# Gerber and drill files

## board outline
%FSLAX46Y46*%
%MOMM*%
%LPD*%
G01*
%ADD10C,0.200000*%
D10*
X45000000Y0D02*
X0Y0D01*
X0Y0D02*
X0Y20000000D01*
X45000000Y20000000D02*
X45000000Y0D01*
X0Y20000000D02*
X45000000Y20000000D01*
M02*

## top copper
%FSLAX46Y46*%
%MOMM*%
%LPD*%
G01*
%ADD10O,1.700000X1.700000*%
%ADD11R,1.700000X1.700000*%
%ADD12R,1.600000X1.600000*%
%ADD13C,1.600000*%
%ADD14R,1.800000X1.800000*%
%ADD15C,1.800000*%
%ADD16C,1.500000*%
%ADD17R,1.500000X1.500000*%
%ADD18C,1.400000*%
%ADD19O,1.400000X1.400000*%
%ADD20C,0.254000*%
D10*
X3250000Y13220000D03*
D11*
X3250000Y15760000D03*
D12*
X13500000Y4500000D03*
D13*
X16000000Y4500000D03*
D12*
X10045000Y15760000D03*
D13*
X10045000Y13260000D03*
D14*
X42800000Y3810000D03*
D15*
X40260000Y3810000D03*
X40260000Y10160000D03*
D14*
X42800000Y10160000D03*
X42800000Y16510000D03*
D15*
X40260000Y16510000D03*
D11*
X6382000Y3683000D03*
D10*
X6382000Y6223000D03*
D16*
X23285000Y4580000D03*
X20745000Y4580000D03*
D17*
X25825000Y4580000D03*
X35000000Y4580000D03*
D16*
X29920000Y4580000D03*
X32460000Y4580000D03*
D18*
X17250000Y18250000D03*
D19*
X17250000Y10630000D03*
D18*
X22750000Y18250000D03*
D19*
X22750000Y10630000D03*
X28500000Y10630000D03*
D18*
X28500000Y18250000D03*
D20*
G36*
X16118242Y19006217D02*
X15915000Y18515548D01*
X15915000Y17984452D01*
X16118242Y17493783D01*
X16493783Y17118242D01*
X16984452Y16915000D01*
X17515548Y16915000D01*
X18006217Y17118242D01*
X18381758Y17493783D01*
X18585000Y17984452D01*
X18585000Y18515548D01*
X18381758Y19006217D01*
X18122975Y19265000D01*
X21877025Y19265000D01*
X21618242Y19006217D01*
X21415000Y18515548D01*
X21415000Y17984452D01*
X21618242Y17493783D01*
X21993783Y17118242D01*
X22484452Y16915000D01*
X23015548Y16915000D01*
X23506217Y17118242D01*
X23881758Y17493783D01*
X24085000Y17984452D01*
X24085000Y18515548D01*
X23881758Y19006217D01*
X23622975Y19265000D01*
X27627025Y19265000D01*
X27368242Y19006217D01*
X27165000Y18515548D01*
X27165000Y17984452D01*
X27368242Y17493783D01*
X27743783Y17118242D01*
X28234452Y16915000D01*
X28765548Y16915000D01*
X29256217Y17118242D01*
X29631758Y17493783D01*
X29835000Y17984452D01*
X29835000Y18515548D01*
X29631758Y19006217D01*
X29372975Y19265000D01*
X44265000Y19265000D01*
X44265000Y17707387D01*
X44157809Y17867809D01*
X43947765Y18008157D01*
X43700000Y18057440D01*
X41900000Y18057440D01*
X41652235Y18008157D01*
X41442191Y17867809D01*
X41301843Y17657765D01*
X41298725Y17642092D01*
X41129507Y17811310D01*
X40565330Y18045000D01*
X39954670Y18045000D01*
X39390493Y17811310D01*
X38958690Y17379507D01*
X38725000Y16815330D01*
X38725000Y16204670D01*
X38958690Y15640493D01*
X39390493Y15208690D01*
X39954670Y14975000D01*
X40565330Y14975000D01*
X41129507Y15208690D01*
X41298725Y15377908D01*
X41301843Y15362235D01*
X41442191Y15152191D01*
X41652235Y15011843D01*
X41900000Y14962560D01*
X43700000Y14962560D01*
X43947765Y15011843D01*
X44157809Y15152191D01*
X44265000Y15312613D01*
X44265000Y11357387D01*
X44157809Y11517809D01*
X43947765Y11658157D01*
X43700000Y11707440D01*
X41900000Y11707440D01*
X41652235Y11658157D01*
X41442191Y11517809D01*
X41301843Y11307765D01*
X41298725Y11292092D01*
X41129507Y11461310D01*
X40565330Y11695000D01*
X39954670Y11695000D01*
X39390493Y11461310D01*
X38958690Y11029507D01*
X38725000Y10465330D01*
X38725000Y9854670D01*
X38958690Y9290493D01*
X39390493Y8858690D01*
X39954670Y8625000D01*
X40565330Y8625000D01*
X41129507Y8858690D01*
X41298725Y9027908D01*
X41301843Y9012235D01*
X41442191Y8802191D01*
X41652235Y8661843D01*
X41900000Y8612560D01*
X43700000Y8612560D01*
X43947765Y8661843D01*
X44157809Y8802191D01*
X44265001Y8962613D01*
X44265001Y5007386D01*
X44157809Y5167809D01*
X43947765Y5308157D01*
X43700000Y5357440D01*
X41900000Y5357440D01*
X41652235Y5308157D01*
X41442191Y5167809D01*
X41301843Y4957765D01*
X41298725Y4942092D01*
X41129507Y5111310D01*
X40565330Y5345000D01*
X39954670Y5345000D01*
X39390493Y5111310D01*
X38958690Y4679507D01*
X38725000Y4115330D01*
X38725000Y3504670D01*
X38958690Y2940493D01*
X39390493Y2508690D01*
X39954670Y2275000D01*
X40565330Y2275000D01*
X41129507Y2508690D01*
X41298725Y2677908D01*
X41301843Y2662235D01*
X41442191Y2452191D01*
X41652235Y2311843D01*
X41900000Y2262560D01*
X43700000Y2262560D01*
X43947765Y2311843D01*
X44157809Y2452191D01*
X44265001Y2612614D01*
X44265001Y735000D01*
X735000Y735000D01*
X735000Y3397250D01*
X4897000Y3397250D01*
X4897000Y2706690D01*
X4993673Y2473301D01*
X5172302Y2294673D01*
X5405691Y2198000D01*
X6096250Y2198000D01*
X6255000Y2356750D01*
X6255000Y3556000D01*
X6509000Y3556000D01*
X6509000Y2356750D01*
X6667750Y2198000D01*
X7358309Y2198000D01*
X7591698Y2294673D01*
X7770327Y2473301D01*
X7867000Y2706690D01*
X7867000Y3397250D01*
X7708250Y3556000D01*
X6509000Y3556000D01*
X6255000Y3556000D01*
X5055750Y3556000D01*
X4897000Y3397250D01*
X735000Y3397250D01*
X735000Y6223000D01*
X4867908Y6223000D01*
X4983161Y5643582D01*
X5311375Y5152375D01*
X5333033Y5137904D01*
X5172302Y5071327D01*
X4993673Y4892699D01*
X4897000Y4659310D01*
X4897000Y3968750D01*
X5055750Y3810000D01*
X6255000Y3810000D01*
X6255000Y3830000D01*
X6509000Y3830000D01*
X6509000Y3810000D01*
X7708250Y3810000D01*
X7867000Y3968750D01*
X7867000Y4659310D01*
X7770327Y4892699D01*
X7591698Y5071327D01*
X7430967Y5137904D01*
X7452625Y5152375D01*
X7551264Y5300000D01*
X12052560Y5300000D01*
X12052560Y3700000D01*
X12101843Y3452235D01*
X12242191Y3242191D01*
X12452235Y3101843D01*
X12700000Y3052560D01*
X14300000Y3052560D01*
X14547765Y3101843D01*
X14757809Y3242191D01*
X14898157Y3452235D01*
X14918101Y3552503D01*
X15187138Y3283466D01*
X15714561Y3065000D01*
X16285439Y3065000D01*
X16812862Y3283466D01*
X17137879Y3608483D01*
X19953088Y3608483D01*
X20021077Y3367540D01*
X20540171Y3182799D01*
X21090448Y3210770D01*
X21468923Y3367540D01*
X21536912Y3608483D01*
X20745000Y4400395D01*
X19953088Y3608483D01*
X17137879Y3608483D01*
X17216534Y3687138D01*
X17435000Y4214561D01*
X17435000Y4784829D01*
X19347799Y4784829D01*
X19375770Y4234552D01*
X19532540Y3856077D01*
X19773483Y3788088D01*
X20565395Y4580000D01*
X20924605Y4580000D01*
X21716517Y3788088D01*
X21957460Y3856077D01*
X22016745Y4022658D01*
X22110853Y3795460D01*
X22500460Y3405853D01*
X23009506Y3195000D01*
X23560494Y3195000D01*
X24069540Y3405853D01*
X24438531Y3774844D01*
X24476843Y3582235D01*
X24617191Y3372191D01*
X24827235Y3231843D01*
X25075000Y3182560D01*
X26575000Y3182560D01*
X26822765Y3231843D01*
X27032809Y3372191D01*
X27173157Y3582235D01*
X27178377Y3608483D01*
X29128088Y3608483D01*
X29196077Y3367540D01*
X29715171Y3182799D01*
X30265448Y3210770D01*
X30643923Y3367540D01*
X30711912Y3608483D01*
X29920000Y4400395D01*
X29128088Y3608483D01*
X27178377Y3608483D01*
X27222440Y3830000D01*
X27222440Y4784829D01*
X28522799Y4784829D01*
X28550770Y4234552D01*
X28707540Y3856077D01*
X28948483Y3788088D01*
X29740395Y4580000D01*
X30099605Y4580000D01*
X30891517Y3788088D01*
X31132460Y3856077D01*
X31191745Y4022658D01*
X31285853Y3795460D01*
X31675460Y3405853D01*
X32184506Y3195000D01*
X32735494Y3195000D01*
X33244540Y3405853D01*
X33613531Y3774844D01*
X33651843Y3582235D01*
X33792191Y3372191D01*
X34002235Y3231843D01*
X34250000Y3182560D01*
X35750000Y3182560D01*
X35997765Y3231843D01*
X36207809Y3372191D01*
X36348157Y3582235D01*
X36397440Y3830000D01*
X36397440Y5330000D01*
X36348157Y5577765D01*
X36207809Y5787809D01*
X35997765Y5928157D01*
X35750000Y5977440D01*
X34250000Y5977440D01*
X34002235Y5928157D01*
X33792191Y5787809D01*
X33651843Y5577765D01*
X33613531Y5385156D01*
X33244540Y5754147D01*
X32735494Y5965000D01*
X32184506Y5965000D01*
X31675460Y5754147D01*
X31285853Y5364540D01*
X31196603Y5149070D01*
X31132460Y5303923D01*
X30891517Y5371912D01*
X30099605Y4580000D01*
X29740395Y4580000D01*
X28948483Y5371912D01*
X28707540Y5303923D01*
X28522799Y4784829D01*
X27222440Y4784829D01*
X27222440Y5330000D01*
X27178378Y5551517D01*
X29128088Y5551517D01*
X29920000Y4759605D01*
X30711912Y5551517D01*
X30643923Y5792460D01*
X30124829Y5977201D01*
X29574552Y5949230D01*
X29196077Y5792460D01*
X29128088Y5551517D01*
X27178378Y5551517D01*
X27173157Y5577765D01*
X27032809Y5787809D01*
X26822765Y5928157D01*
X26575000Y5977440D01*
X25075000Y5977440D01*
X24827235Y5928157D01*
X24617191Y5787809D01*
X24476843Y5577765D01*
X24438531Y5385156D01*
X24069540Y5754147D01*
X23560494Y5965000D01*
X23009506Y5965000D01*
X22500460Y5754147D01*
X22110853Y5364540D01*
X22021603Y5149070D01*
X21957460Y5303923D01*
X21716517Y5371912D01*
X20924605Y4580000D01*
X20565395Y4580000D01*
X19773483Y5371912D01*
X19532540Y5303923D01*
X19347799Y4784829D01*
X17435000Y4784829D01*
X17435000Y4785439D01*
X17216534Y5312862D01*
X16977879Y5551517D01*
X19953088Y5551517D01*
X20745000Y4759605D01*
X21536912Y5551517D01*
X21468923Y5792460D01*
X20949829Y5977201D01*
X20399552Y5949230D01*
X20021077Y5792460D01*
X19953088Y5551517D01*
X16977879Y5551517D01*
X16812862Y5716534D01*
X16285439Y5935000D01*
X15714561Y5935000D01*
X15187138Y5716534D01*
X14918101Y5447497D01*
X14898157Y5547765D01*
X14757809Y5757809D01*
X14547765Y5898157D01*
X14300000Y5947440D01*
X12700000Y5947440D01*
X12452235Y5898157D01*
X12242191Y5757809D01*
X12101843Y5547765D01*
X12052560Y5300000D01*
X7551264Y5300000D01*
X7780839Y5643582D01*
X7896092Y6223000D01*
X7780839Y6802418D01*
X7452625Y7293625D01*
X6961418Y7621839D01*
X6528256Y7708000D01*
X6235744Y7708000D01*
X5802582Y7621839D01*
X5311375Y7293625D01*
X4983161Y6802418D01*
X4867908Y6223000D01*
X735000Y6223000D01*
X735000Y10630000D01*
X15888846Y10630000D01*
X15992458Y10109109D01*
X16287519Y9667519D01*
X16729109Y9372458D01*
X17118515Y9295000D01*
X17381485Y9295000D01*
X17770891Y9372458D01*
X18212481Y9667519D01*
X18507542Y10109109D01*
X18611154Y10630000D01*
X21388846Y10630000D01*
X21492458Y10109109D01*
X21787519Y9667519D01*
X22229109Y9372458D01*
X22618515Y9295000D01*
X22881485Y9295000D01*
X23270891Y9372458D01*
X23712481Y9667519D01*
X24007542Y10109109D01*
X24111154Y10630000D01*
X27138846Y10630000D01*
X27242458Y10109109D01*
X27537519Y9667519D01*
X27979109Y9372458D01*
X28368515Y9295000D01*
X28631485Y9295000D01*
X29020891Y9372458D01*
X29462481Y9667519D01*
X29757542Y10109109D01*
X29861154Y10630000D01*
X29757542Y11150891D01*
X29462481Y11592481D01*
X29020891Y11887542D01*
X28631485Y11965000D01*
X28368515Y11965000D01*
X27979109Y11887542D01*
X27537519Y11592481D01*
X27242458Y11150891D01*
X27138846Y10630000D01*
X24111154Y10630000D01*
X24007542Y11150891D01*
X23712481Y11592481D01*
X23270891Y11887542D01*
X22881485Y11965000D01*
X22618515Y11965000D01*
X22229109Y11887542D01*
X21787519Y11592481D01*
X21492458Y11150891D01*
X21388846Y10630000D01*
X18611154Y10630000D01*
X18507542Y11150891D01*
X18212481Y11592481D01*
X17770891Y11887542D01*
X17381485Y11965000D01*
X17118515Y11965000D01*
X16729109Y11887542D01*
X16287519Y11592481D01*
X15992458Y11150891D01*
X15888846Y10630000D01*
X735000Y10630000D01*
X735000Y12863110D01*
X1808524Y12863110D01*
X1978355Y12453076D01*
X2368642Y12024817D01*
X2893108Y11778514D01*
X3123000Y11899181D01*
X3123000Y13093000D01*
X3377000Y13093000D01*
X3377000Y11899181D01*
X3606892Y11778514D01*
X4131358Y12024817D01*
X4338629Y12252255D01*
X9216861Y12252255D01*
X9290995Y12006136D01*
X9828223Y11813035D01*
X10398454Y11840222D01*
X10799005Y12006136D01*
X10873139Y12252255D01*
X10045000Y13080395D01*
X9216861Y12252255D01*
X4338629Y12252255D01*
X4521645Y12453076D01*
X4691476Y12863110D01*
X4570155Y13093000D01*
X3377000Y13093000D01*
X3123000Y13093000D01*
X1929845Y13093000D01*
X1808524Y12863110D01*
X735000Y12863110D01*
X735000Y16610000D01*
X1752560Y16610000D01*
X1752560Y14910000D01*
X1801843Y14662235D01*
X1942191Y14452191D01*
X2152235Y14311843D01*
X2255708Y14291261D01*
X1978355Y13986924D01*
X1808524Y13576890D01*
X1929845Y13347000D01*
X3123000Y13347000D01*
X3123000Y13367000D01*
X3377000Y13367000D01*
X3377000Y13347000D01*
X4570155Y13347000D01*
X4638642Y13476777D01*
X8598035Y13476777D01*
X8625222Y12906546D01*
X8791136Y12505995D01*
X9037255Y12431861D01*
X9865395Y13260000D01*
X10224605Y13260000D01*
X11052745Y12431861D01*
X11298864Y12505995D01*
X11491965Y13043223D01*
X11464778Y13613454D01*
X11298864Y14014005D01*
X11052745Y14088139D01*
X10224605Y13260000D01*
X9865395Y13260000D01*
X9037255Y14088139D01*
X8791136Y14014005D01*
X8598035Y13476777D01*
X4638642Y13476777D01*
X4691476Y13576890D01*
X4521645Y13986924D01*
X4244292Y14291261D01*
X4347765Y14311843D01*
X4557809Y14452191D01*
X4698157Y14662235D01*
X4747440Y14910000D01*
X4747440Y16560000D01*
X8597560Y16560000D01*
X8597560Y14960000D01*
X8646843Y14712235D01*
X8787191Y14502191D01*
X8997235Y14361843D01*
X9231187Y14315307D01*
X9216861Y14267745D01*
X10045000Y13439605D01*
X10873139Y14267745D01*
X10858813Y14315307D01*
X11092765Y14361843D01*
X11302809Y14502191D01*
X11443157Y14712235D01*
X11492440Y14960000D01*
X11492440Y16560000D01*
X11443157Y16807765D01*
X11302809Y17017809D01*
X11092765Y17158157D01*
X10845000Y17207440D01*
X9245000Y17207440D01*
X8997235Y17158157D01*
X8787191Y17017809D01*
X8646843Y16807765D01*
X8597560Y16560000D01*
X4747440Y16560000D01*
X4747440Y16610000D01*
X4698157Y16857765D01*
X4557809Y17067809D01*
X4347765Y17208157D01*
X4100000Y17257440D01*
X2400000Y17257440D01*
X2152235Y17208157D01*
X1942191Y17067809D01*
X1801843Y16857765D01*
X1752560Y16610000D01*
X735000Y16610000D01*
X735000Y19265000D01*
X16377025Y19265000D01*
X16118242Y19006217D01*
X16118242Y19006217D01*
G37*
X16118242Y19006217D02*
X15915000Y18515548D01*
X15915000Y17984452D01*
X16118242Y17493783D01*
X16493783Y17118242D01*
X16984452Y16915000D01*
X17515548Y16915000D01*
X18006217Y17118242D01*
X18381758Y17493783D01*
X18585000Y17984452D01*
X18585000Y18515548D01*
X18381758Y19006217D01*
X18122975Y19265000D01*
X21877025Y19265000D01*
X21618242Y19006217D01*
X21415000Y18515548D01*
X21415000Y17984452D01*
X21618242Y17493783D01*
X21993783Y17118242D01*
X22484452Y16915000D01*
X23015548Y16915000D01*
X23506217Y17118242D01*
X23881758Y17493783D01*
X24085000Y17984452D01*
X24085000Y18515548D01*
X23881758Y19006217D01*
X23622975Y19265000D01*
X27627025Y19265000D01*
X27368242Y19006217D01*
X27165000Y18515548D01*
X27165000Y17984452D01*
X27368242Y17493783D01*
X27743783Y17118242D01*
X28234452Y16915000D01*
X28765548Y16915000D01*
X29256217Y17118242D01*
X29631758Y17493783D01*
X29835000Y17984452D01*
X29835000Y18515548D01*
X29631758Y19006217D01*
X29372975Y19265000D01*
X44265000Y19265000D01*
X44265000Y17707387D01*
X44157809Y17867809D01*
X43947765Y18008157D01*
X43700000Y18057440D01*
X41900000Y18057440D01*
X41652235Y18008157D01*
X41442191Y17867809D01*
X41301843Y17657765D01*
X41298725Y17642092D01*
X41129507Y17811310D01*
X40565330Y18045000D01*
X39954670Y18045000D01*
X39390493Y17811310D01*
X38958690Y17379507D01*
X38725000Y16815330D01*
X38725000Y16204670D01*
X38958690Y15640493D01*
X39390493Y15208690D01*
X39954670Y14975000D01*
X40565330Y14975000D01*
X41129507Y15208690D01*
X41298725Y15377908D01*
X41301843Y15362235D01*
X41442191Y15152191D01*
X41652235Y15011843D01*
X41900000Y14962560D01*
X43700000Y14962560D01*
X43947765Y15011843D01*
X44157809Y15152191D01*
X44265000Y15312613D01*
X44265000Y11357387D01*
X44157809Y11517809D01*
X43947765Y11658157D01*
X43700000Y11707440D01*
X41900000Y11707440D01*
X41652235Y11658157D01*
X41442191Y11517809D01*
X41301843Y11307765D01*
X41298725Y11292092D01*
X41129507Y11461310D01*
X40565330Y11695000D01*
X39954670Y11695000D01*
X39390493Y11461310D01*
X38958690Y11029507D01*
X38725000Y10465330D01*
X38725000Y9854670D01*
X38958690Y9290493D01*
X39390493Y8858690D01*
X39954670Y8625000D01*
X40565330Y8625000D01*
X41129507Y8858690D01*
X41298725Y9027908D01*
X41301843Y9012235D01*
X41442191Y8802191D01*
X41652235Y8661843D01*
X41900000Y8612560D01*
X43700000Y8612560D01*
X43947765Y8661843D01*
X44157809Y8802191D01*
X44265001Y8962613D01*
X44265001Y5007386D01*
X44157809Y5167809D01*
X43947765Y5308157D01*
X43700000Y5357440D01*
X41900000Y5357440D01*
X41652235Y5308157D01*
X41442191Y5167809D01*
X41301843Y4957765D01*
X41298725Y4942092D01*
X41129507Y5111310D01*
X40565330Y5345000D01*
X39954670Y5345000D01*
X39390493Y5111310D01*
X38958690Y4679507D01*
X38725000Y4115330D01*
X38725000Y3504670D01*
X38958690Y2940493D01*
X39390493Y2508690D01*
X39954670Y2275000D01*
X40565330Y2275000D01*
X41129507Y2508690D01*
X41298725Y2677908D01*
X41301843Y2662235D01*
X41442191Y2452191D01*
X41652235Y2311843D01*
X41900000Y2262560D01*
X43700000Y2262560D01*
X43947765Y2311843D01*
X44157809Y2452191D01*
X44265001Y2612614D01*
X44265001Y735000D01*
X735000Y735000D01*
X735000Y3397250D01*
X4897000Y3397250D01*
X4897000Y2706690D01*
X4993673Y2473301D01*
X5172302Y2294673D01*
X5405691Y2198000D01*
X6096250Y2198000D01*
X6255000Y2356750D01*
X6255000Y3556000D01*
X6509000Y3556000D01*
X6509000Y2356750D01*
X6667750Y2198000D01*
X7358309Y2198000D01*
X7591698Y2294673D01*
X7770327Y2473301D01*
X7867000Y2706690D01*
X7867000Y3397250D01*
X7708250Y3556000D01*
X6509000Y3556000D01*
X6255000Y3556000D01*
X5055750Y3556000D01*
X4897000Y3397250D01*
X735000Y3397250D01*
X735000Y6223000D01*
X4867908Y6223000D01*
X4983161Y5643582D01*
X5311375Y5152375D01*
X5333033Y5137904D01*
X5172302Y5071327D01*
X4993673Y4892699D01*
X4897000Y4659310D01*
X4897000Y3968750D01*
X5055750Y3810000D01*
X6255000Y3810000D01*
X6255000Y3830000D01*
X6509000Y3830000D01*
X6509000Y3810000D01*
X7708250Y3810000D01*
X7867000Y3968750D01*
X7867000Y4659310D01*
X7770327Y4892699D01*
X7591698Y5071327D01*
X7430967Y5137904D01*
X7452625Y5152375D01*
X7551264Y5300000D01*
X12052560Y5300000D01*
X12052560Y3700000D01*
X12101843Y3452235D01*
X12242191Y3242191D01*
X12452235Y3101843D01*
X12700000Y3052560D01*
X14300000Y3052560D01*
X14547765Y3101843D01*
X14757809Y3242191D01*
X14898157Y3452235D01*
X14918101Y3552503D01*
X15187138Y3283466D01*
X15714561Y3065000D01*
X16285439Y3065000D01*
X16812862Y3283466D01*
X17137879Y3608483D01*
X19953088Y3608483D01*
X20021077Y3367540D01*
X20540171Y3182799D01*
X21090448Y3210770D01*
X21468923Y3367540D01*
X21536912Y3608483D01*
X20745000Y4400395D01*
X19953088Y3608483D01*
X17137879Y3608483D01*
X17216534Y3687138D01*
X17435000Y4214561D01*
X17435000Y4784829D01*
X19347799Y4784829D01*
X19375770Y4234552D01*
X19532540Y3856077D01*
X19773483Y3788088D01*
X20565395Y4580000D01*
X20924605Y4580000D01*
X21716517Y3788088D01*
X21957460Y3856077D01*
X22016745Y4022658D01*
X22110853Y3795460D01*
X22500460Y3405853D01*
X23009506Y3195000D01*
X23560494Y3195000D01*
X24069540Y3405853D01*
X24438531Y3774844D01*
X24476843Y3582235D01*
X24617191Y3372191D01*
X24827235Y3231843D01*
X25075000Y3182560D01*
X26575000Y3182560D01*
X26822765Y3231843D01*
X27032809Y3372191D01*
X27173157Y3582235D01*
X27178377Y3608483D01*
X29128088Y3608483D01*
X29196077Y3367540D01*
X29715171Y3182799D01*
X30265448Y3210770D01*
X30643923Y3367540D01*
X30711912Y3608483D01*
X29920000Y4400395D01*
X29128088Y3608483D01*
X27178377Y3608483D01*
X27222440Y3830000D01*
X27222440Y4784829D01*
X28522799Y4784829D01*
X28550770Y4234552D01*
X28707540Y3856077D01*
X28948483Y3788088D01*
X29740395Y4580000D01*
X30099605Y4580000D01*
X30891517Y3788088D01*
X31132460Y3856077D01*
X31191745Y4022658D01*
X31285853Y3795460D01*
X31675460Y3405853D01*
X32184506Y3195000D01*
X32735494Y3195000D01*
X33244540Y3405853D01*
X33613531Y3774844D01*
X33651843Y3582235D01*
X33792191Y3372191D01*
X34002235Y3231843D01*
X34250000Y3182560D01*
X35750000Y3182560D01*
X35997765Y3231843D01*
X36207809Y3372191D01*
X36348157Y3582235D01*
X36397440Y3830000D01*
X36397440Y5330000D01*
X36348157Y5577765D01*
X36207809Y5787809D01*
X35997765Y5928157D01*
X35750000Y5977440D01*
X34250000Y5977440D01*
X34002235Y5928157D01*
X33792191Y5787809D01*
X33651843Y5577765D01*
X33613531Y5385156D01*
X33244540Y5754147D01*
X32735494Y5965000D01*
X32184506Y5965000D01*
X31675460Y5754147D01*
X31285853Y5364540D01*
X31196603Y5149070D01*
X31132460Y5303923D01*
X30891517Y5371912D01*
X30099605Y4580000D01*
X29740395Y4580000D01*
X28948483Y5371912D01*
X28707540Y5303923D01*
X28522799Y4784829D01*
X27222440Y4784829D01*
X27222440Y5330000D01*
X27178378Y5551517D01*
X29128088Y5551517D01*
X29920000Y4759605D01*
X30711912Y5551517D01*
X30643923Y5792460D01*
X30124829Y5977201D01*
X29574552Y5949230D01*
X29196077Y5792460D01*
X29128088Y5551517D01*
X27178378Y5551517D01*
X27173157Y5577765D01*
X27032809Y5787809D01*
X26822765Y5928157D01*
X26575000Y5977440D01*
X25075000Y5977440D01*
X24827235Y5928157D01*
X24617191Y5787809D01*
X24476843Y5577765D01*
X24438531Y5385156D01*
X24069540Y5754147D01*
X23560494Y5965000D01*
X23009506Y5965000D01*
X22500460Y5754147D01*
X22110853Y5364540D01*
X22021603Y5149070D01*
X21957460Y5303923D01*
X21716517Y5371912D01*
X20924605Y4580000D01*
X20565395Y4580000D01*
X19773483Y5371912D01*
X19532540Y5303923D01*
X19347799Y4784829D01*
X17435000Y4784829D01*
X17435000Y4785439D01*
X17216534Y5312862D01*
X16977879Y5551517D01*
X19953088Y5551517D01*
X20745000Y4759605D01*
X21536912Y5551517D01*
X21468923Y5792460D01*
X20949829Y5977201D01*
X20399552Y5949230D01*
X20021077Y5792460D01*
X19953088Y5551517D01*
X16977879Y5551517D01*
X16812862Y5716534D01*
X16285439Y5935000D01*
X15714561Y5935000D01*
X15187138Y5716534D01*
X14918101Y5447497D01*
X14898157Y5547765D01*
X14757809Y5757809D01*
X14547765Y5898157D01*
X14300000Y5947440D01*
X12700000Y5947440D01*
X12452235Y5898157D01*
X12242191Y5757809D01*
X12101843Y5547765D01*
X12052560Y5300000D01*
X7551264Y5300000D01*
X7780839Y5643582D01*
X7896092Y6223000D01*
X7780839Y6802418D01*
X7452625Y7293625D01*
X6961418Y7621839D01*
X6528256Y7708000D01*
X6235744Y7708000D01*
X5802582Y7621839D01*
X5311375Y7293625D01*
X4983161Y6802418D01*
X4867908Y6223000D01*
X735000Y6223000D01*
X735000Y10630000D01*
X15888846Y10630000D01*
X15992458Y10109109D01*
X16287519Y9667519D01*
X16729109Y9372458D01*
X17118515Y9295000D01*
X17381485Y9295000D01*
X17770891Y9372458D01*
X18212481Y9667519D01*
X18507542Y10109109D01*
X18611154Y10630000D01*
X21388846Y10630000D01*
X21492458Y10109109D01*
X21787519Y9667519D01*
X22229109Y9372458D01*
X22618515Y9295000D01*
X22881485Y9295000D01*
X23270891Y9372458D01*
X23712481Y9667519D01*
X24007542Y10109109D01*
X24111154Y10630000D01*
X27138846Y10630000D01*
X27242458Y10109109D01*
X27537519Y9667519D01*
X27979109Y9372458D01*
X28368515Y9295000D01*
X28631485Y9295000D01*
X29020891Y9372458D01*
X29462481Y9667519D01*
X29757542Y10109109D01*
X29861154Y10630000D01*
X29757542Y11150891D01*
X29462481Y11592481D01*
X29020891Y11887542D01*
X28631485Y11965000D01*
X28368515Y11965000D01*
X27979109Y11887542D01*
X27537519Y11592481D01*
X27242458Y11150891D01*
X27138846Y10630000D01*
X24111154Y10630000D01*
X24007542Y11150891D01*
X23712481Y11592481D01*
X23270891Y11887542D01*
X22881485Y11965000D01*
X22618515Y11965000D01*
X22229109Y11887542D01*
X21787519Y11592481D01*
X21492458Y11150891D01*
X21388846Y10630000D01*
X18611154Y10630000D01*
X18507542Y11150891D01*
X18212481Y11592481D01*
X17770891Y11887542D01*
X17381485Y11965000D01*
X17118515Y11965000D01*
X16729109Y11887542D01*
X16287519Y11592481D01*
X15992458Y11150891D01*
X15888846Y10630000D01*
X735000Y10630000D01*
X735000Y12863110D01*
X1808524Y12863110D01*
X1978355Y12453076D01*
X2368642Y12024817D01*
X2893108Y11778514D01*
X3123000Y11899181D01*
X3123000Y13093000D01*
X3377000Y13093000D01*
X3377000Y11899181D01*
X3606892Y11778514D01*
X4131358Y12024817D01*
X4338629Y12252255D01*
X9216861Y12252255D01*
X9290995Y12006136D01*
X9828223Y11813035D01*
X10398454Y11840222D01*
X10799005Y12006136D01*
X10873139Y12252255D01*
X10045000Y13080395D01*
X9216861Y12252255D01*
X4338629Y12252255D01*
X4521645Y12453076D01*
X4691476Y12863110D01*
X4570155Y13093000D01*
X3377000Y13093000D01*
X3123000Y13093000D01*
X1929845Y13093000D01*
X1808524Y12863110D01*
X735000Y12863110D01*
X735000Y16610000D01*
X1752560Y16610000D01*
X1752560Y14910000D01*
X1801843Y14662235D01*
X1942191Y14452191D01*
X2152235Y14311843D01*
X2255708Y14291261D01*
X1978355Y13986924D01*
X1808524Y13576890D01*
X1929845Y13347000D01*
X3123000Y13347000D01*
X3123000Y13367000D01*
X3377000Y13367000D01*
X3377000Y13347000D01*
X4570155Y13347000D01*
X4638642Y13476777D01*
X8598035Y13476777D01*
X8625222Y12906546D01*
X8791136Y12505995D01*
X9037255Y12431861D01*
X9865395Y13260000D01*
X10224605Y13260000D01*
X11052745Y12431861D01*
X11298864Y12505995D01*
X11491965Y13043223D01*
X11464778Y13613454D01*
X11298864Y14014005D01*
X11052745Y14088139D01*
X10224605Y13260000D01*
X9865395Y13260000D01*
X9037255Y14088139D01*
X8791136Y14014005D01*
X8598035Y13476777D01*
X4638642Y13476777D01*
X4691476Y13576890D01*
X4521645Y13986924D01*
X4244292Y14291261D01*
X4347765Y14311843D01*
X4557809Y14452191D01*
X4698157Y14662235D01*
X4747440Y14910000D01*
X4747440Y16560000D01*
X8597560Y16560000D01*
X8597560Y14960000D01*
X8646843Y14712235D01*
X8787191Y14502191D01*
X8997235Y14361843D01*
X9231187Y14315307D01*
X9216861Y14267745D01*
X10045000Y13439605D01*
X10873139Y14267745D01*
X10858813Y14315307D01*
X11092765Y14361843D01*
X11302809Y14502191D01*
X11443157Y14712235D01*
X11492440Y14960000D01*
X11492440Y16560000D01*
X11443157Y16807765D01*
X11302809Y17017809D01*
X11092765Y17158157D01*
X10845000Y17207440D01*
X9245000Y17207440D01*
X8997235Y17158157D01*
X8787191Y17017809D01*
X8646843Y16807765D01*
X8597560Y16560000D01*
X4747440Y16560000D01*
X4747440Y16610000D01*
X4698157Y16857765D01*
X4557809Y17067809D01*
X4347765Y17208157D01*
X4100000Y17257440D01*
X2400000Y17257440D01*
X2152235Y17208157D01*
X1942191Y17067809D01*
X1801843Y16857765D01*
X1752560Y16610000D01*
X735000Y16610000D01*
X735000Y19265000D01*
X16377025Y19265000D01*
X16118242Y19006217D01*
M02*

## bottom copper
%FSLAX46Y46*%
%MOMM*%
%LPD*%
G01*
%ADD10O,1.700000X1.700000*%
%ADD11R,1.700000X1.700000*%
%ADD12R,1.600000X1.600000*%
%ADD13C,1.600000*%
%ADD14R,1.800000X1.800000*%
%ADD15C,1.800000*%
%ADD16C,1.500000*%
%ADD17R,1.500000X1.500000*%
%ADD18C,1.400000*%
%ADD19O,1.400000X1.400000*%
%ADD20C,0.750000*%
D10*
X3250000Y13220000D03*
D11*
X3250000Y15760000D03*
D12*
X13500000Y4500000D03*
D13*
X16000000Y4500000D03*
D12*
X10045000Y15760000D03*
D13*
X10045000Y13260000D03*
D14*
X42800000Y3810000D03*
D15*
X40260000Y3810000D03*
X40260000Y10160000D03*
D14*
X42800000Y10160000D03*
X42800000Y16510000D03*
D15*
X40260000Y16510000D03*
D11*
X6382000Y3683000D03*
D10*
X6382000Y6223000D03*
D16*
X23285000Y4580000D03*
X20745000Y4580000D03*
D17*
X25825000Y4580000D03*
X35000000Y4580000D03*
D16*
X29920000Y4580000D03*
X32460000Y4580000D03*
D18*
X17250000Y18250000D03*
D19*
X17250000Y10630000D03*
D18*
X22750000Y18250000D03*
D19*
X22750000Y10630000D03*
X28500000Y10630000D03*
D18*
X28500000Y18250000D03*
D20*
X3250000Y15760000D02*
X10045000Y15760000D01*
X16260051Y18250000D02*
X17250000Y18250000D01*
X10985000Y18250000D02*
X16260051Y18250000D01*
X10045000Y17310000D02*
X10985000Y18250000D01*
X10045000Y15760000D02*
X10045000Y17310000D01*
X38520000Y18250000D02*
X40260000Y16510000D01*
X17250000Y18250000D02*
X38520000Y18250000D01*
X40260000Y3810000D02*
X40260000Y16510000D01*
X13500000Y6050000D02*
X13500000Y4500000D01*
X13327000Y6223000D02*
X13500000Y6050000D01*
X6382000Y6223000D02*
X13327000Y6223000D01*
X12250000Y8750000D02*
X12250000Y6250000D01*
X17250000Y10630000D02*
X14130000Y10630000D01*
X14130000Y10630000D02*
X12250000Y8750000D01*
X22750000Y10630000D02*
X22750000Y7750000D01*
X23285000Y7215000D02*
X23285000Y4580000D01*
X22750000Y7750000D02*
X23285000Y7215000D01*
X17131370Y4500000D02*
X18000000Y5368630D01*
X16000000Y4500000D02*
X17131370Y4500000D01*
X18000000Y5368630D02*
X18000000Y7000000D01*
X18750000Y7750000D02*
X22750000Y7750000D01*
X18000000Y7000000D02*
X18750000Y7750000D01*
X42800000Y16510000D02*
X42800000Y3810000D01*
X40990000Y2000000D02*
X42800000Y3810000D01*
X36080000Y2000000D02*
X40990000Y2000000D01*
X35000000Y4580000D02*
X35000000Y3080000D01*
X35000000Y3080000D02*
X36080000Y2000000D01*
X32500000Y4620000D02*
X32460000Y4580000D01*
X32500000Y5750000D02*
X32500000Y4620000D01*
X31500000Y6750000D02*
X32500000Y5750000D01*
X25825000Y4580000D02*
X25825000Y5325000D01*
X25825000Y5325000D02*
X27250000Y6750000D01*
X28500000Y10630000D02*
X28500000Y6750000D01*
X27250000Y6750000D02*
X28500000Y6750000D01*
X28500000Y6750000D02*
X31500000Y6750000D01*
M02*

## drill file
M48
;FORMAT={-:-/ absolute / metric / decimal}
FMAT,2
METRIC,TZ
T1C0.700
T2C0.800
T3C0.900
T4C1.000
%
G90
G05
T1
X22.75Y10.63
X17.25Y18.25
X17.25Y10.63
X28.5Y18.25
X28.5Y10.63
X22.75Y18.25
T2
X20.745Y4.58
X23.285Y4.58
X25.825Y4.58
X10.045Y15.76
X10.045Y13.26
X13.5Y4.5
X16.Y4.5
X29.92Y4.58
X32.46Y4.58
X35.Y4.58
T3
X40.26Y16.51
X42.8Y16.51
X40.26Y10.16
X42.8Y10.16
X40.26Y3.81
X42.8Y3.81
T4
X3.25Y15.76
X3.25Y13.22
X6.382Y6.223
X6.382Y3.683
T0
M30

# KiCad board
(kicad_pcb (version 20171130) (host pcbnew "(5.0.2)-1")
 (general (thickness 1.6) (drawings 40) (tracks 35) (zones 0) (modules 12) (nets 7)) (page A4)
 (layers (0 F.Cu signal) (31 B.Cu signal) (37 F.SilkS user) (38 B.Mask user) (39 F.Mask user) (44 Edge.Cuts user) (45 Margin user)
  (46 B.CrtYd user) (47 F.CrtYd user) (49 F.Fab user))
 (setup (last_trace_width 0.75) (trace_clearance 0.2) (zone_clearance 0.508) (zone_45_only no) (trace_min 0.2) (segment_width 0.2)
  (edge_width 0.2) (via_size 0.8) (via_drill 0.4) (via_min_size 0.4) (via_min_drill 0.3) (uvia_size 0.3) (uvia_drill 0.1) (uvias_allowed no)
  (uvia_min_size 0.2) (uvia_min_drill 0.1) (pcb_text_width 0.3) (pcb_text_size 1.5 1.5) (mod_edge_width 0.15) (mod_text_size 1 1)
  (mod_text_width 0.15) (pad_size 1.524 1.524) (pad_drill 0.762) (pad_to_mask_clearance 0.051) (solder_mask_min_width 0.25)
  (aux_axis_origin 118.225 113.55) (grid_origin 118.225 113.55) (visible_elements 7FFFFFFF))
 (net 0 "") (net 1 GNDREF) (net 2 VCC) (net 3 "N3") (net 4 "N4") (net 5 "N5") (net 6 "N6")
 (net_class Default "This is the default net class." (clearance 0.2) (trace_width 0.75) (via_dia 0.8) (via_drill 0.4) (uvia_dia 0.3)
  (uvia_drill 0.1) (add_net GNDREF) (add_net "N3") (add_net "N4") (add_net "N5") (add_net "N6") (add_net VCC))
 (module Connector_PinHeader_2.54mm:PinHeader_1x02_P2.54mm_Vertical (layer F.Cu) (at 121.475 97.79)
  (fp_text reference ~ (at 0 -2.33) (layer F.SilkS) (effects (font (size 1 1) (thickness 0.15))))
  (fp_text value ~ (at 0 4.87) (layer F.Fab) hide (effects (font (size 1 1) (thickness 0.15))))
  (pad 2 thru_hole oval (at 0 2.54) (size 1.7 1.7) (drill 1) (layers *.Cu *.Mask) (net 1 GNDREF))
  (pad 1 thru_hole rect (at 0 0) (size 1.7 1.7) (drill 1) (layers *.Cu *.Mask) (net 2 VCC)))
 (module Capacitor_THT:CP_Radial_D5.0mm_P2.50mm (layer F.Cu) (at 131.725 109.05)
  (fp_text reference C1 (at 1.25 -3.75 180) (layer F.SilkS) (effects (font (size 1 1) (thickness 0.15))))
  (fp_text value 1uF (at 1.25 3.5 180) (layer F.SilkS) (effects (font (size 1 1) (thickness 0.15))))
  (pad 1 thru_hole rect (at 0 0) (size 1.6 1.6) (drill 0.8) (layers *.Cu *.Mask) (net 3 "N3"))
  (pad 2 thru_hole circle (at 2.5 0) (size 1.6 1.6) (drill 0.8) (layers *.Cu *.Mask) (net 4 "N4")))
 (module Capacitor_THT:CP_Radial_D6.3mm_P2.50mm (layer F.Cu) (at 128.27 97.79 270)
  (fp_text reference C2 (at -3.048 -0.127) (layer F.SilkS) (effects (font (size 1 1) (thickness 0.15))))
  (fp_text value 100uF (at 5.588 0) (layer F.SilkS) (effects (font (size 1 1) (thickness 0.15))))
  (pad 1 thru_hole rect (at 0 0 270) (size 1.6 1.6) (drill 0.8) (layers *.Cu *.Mask) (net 2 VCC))
  (pad 2 thru_hole circle (at 2.5 0 270) (size 1.6 1.6) (drill 0.8) (layers *.Cu *.Mask) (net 1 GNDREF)))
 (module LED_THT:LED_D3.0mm (layer F.Cu) (at 161.025 109.74 180)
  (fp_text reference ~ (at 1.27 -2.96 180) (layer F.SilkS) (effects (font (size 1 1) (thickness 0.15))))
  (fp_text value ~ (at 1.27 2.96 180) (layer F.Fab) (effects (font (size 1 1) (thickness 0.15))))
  (pad 1 thru_hole rect (at 0 0 180) (size 1.8 1.8) (drill 0.9) (layers *.Cu *.Mask) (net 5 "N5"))
  (pad 2 thru_hole circle (at 2.54 0 180) (size 1.8 1.8) (drill 0.9) (layers *.Cu *.Mask) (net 2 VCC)))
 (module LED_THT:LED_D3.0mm (layer F.Cu) (at 161.025 103.39 180)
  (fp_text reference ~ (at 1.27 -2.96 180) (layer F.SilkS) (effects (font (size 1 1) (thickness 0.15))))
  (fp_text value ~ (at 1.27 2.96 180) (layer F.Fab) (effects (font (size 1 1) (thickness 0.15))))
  (pad 2 thru_hole circle (at 2.54 0 180) (size 1.8 1.8) (drill 0.9) (layers *.Cu *.Mask) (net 2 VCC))
  (pad 1 thru_hole rect (at 0 0 180) (size 1.8 1.8) (drill 0.9) (layers *.Cu *.Mask) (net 5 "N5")))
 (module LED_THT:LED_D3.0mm (layer F.Cu) (at 161.025 97.04 180)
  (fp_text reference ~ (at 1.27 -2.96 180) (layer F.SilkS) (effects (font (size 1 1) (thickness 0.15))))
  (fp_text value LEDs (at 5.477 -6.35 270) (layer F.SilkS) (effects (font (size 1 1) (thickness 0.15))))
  (pad 1 thru_hole rect (at 0 0 180) (size 1.8 1.8) (drill 0.9) (layers *.Cu *.Mask) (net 5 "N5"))
  (pad 2 thru_hole circle (at 2.54 0 180) (size 1.8 1.8) (drill 0.9) (layers *.Cu *.Mask) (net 2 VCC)))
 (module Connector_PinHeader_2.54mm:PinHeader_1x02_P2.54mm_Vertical (layer F.Cu) (at 124.607 109.867 180)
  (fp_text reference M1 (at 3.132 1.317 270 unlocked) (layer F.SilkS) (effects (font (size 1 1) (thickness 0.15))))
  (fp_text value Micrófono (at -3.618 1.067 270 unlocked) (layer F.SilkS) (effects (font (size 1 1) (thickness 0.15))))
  (pad 1 thru_hole rect (at 0 0 180) (size 1.7 1.7) (drill 1) (layers *.Cu *.Mask) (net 1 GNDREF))
  (pad 2 thru_hole oval (at 0 2.54 180) (size 1.7 1.7) (drill 1) (layers *.Cu *.Mask) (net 3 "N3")))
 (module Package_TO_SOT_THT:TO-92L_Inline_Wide (layer F.Cu) (at 144.05 108.97 180)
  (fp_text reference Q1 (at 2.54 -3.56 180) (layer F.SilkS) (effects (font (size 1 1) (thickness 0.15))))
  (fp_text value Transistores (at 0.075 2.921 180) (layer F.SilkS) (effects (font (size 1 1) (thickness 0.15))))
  (pad 2 thru_hole circle (at 2.54 0 270) (size 1.5 1.5) (drill 0.8) (layers *.Cu *.Mask) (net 4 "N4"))
  (pad 3 thru_hole circle (at 5.08 0 270) (size 1.5 1.5) (drill 0.8) (layers *.Cu *.Mask) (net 1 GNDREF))
  (pad 1 thru_hole rect (at 0 0 270) (size 1.5 1.5) (drill 0.8) (layers *.Cu *.Mask) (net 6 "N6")))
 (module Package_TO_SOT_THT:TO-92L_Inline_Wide (layer F.Cu) (at 153.225 108.97 180)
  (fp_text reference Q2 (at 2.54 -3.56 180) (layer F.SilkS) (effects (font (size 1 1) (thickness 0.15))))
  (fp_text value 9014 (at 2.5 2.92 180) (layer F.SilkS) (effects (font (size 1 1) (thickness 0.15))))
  (pad 1 thru_hole rect (at 0 0 270) (size 1.5 1.5) (drill 0.8) (layers *.Cu *.Mask) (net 5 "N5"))
  (pad 3 thru_hole circle (at 5.08 0 270) (size 1.5 1.5) (drill 0.8) (layers *.Cu *.Mask) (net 1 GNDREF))
  (pad 2 thru_hole circle (at 2.54 0 270) (size 1.5 1.5) (drill 0.8) (layers *.Cu *.Mask) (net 6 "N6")))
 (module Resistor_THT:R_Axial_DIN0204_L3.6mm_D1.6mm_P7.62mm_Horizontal (layer F.Cu) (at 135.475 95.3 270)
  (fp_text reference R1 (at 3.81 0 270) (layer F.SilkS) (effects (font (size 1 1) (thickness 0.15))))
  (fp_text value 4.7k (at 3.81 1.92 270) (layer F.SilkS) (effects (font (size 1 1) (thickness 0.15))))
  (pad 1 thru_hole circle (at 0 0 270) (size 1.4 1.4) (drill 0.7) (layers *.Cu *.Mask) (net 2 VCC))
  (pad 2 thru_hole oval (at 7.62 0 270) (size 1.4 1.4) (drill 0.7) (layers *.Cu *.Mask) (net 3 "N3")))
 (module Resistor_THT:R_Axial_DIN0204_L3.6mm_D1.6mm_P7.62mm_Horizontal (layer F.Cu) (at 140.975 95.3 270)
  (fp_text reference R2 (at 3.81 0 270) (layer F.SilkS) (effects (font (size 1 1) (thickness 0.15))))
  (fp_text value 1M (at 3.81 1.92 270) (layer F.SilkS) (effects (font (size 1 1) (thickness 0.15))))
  (pad 1 thru_hole circle (at 0 0 270) (size 1.4 1.4) (drill 0.7) (layers *.Cu *.Mask) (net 2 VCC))
  (pad 2 thru_hole oval (at 7.62 0 270) (size 1.4 1.4) (drill 0.7) (layers *.Cu *.Mask) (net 4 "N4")))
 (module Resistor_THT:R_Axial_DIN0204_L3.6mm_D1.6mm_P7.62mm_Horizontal (layer F.Cu) (at 146.725 95.3 270)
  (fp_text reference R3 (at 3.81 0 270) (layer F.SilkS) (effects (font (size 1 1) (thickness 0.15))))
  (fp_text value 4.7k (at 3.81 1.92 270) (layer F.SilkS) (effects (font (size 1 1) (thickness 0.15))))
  (pad 2 thru_hole oval (at 7.62 0 270) (size 1.4 1.4) (drill 0.7) (layers *.Cu *.Mask) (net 6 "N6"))
  (pad 1 thru_hole circle (at 0 0 270) (size 1.4 1.4) (drill 0.7) (layers *.Cu *.Mask) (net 2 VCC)))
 (gr_line (start 163.225 113.55) (end 118.225 113.55) (layer Edge.Cuts) (width 0.2))
 (gr_line (start 118.225 113.55) (end 118.225 93.55) (layer Edge.Cuts) (width 0.2))
 (gr_line (start 163.225 93.55) (end 163.225 113.55) (layer Edge.Cuts) (width 0.2))
 (gr_line (start 118.225 93.55) (end 163.225 93.55) (layer Edge.Cuts) (width 0.2))
 (segment (start 121.475 97.79) (end 128.27 97.79) (width 0.75) (layer B.Cu) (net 2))
 (segment (start 134.485051 95.3) (end 135.475 95.3) (width 0.75) (layer B.Cu) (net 2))
 (segment (start 129.21 95.3) (end 134.485051 95.3) (width 0.75) (layer B.Cu) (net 2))
 (segment (start 128.27 96.24) (end 129.21 95.3) (width 0.75) (layer B.Cu) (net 2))
 (segment (start 128.27 97.79) (end 128.27 96.24) (width 0.75) (layer B.Cu) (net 2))
 (segment (start 156.745 95.3) (end 158.485 97.04) (width 0.75) (layer B.Cu) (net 2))
 (segment (start 135.475 95.3) (end 156.745 95.3) (width 0.75) (layer B.Cu) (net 2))
 (segment (start 158.485 109.74) (end 158.485 97.04) (width 0.75) (layer B.Cu) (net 2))
 (segment (start 131.725 107.5) (end 131.725 109.05) (width 0.75) (layer B.Cu) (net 3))
 (segment (start 131.552 107.327) (end 131.725 107.5) (width 0.75) (layer B.Cu) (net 3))
 (segment (start 124.607 107.327) (end 131.552 107.327) (width 0.75) (layer B.Cu) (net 3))
 (segment (start 130.475 104.8) (end 130.475 107.3) (width 0.75) (layer B.Cu) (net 3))
 (segment (start 135.475 102.92) (end 132.355 102.92) (width 0.75) (layer B.Cu) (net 3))
 (segment (start 132.355 102.92) (end 130.475 104.8) (width 0.75) (layer B.Cu) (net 3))
 (segment (start 140.975 102.92) (end 140.975 105.8) (width 0.75) (layer B.Cu) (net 4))
 (segment (start 141.51 106.335) (end 141.51 108.97) (width 0.75) (layer B.Cu) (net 4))
 (segment (start 140.975 105.8) (end 141.51 106.335) (width 0.75) (layer B.Cu) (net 4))
 (segment (start 135.35637 109.05) (end 136.225 108.18137) (width 0.75) (layer B.Cu) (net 4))
 (segment (start 134.225 109.05) (end 135.35637 109.05) (width 0.75) (layer B.Cu) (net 4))
 (segment (start 136.225 108.18137) (end 136.225 106.55) (width 0.75) (layer B.Cu) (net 4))
 (segment (start 136.975 105.8) (end 140.975 105.8) (width 0.75) (layer B.Cu) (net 4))
 (segment (start 136.225 106.55) (end 136.975 105.8) (width 0.75) (layer B.Cu) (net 4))
 (segment (start 161.025 97.04) (end 161.025 109.74) (width 0.75) (layer B.Cu) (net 5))
 (segment (start 159.215 111.55) (end 161.025 109.74) (width 0.75) (layer B.Cu) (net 5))
 (segment (start 154.305 111.55) (end 159.215 111.55) (width 0.75) (layer B.Cu) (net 5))
 (segment (start 153.225 108.97) (end 153.225 110.47) (width 0.75) (layer B.Cu) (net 5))
 (segment (start 153.225 110.47) (end 154.305 111.55) (width 0.75) (layer B.Cu) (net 5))
 (segment (start 150.725 108.93) (end 150.685 108.97) (width 0.75) (layer B.Cu) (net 6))
 (segment (start 150.725 107.8) (end 150.725 108.93) (width 0.75) (layer B.Cu) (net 6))
 (segment (start 149.725 106.8) (end 150.725 107.8) (width 0.75) (layer B.Cu) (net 6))
 (segment (start 144.05 108.97) (end 144.05 108.225) (width 0.75) (layer B.Cu) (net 6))
 (segment (start 144.05 108.225) (end 145.475 106.8) (width 0.75) (layer B.Cu) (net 6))
 (segment (start 146.725 102.92) (end 146.725 106.8) (width 0.75) (layer B.Cu) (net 6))
 (segment (start 145.475 106.8) (end 146.725 106.8) (width 0.75) (layer B.Cu) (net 6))
 (segment (start 146.725 106.8) (end 149.725 106.8) (width 0.75) (layer B.Cu) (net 6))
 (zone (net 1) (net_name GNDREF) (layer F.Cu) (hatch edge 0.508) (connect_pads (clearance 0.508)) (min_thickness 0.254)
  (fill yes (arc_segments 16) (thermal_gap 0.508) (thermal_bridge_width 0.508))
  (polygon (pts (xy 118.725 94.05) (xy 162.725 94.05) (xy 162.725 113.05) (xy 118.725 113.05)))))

